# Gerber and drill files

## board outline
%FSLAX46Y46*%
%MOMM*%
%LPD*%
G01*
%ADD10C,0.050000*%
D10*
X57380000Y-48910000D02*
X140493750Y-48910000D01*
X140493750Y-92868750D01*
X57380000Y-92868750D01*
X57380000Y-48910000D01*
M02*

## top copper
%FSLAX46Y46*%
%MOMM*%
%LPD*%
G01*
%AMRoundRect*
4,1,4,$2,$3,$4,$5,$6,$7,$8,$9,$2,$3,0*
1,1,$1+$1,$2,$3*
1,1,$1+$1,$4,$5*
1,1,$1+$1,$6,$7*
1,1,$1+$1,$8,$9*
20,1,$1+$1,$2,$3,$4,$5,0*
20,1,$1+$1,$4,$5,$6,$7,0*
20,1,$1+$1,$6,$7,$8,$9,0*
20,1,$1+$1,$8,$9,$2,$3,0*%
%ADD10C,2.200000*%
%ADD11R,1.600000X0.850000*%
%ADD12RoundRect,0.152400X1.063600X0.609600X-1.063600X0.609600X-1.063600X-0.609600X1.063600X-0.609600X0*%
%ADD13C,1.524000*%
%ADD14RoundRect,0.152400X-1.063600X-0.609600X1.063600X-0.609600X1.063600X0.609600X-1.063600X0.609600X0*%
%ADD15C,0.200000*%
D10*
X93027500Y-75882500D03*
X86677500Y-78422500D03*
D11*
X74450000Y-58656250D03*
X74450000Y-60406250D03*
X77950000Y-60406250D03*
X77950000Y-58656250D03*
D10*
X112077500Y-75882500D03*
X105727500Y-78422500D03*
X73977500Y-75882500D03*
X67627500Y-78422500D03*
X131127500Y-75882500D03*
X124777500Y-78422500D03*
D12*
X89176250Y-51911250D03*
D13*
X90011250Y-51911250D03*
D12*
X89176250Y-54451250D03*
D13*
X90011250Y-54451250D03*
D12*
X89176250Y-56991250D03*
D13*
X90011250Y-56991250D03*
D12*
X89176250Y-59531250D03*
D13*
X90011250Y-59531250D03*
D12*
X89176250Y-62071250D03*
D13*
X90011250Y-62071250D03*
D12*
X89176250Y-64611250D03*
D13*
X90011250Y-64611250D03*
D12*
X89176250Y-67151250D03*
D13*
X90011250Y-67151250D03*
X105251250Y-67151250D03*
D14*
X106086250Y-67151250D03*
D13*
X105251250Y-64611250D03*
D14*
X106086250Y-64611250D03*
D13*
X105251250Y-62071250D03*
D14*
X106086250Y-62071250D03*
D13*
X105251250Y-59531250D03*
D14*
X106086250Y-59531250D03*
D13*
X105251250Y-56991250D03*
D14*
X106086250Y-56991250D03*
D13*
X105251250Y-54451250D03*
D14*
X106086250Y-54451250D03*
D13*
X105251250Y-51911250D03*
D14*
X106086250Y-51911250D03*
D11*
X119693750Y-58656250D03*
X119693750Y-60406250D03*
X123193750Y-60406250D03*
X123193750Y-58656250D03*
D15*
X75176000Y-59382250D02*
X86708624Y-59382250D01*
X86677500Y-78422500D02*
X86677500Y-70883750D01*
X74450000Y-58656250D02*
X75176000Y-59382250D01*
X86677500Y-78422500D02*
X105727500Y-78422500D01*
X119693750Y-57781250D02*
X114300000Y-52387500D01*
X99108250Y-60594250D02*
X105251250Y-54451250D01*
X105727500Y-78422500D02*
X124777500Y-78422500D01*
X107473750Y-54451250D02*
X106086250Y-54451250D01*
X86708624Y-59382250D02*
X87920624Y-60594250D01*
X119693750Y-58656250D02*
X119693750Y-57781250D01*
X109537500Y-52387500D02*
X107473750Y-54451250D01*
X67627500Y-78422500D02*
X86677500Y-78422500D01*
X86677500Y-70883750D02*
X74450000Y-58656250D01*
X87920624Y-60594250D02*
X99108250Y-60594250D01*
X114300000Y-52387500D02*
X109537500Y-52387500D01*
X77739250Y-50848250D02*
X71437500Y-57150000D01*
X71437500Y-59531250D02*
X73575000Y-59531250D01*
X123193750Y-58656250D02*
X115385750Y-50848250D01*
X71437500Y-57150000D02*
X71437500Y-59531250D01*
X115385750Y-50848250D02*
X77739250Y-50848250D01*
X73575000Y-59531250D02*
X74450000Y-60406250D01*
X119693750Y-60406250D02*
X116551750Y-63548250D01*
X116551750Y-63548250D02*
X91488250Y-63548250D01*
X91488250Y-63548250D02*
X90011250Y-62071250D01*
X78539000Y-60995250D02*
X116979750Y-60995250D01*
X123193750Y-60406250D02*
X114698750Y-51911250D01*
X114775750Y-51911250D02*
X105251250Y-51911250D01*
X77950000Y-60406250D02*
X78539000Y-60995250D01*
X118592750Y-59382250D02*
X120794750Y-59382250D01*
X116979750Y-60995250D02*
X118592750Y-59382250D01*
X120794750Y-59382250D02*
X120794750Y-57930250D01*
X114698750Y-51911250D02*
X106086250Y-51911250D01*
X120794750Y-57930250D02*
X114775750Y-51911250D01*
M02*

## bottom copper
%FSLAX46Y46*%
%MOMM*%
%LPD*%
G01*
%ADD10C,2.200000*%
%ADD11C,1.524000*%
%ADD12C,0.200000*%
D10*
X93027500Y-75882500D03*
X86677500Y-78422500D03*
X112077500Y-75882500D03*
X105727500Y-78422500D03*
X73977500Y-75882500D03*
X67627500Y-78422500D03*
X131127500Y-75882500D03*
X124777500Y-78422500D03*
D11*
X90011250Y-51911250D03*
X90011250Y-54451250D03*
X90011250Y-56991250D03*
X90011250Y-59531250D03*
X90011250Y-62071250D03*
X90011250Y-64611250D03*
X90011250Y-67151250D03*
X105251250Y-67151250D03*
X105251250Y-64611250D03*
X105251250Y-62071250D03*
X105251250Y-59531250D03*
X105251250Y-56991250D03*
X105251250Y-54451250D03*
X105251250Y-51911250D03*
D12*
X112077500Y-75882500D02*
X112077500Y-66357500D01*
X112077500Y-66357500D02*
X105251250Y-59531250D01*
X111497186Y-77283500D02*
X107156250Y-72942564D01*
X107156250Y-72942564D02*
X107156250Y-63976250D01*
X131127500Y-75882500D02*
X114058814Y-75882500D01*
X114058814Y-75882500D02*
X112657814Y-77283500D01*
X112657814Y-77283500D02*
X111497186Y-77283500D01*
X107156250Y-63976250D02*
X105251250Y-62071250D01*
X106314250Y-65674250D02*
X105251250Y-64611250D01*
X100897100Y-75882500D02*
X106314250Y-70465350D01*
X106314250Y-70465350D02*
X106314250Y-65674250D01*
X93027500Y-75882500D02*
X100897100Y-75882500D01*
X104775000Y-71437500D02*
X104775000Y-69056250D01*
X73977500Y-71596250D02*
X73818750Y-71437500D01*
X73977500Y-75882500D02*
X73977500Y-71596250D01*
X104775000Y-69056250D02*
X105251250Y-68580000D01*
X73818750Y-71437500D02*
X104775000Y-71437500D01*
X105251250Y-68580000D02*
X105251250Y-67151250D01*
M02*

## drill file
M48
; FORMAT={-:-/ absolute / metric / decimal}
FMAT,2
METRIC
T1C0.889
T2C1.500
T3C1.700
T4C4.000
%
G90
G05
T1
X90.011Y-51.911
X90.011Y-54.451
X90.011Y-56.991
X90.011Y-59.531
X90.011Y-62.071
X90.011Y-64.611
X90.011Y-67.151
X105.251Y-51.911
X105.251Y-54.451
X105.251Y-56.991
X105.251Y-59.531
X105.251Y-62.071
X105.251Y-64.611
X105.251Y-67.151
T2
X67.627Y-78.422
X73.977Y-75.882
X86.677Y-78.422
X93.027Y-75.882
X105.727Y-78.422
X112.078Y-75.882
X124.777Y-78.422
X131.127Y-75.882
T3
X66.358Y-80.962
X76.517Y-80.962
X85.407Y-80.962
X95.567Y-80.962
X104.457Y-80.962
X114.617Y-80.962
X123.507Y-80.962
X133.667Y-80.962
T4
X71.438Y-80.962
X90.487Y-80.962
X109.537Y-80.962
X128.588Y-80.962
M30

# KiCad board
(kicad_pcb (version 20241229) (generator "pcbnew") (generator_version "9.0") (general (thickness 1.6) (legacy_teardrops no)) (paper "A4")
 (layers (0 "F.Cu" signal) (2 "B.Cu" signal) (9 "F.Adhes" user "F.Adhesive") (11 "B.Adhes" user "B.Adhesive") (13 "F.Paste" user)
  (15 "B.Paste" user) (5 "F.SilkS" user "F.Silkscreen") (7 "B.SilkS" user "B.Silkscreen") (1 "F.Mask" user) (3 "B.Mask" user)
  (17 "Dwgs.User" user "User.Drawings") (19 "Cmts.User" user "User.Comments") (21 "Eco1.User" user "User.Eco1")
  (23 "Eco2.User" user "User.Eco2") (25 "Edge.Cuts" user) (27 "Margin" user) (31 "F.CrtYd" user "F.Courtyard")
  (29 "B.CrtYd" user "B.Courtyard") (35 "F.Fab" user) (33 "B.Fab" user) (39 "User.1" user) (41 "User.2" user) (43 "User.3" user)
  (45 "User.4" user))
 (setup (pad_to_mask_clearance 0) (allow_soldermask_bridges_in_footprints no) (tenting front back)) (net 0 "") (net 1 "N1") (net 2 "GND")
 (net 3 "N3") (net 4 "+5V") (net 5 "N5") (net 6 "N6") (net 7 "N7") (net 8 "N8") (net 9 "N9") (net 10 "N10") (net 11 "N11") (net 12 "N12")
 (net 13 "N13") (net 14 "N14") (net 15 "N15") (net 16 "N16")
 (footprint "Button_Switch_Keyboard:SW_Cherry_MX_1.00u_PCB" (layer "F.Cu") (at 93.0275 75.8825)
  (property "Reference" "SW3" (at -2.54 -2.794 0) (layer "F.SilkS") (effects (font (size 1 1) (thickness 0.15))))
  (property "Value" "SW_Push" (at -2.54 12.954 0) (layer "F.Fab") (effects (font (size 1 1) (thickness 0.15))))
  (pad "" np_thru_hole circle (at -7.62 5.08) (size 1.7 1.7) (drill 1.7) (layers "*.Cu" "*.Mask"))
  (pad "" np_thru_hole circle (at -2.54 5.08) (size 4 4) (drill 4) (layers "*.Cu" "*.Mask"))
  (pad "" np_thru_hole circle (at 2.54 5.08) (size 1.7 1.7) (drill 1.7) (layers "*.Cu" "*.Mask"))
  (pad "1" thru_hole circle (at 0 0) (size 2.2 2.2) (drill 1.5) (layers "*.Cu" "*.Mask") (remove_unused_layers no) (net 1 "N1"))
  (pad "2" thru_hole circle (at -6.35 2.54) (size 2.2 2.2) (drill 1.5) (layers "*.Cu" "*.Mask") (remove_unused_layers no) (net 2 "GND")))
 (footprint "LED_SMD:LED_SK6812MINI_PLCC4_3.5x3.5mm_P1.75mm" (layer "F.Cu") (at 76.2 59.53125)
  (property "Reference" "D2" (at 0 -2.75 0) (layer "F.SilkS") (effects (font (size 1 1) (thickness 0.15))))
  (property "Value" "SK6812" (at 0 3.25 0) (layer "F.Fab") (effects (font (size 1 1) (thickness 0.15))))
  (pad "1" smd rect (at -1.75 -0.875) (size 1.6 0.85) (layers "F.Cu" "F.Mask" "F.Paste") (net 2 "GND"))
  (pad "2" smd rect (at -1.75 0.875) (size 1.6 0.85) (layers "F.Cu" "F.Mask" "F.Paste") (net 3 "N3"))
  (pad "3" smd rect (at 1.75 0.875) (size 1.6 0.85) (layers "F.Cu" "F.Mask" "F.Paste") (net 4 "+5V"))
  (pad "4" smd rect (at 1.75 -0.875) (size 1.6 0.85) (layers "F.Cu" "F.Mask" "F.Paste") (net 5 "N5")))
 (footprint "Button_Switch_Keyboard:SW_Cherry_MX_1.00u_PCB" (layer "F.Cu") (at 112.0775 75.8825)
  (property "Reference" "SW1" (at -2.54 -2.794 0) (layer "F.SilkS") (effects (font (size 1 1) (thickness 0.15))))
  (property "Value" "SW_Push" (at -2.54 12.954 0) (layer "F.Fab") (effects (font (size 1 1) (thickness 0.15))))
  (pad "" np_thru_hole circle (at -7.62 5.08) (size 1.7 1.7) (drill 1.7) (layers "*.Cu" "*.Mask"))
  (pad "" np_thru_hole circle (at -2.54 5.08) (size 4 4) (drill 4) (layers "*.Cu" "*.Mask"))
  (pad "" np_thru_hole circle (at 2.54 5.08) (size 1.7 1.7) (drill 1.7) (layers "*.Cu" "*.Mask"))
  (pad "1" thru_hole circle (at 0 0) (size 2.2 2.2) (drill 1.5) (layers "*.Cu" "*.Mask") (remove_unused_layers no) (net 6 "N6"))
  (pad "2" thru_hole circle (at -6.35 2.54) (size 2.2 2.2) (drill 1.5) (layers "*.Cu" "*.Mask") (remove_unused_layers no) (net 2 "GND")))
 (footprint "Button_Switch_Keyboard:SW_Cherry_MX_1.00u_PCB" (layer "F.Cu") (at 73.9775 75.8825)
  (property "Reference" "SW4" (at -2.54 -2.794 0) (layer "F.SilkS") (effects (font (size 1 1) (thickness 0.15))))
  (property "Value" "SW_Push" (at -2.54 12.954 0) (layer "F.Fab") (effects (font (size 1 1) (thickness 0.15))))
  (pad "" np_thru_hole circle (at -7.62 5.08) (size 1.7 1.7) (drill 1.7) (layers "*.Cu" "*.Mask"))
  (pad "" np_thru_hole circle (at -2.54 5.08) (size 4 4) (drill 4) (layers "*.Cu" "*.Mask"))
  (pad "" np_thru_hole circle (at 2.54 5.08) (size 1.7 1.7) (drill 1.7) (layers "*.Cu" "*.Mask"))
  (pad "1" thru_hole circle (at 0 0) (size 2.2 2.2) (drill 1.5) (layers "*.Cu" "*.Mask") (remove_unused_layers no) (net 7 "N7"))
  (pad "2" thru_hole circle (at -6.35 2.54) (size 2.2 2.2) (drill 1.5) (layers "*.Cu" "*.Mask") (remove_unused_layers no) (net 2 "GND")))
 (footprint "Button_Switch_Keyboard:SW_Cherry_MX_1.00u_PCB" (layer "F.Cu") (at 131.1275 75.8825)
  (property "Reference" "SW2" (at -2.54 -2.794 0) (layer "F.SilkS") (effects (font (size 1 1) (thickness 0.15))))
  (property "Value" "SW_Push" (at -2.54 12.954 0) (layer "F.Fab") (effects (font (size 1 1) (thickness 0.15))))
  (pad "" np_thru_hole circle (at -7.62 5.08) (size 1.7 1.7) (drill 1.7) (layers "*.Cu" "*.Mask"))
  (pad "" np_thru_hole circle (at -2.54 5.08) (size 4 4) (drill 4) (layers "*.Cu" "*.Mask"))
  (pad "" np_thru_hole circle (at 2.54 5.08) (size 1.7 1.7) (drill 1.7) (layers "*.Cu" "*.Mask"))
  (pad "1" thru_hole circle (at 0 0) (size 2.2 2.2) (drill 1.5) (layers "*.Cu" "*.Mask") (remove_unused_layers no) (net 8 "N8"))
  (pad "2" thru_hole circle (at -6.35 2.54) (size 2.2 2.2) (drill 1.5) (layers "*.Cu" "*.Mask") (remove_unused_layers no) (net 2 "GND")))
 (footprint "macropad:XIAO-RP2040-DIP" (layer "F.Cu") (at 97.63125 59.53125)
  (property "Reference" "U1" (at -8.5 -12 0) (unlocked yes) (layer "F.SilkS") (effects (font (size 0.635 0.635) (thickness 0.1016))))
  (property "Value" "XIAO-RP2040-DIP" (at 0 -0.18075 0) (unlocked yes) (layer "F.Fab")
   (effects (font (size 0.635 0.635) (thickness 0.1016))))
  (pad "1" smd roundrect (at -8.455 -7.62 180) (size 2.432 1.524) (layers "F.Cu" "F.Mask") (roundrect_rratio 0.1) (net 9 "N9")
   (thermal_bridge_angle 45))
  (pad "1" thru_hole circle (at -7.62 -7.62 180) (size 1.524 1.524) (drill 0.889) (layers "*.Cu" "*.Mask") (remove_unused_layers no)
   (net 9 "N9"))
  (pad "2" smd roundrect (at -8.455 -5.08 180) (size 2.432 1.524) (layers "F.Cu" "F.Mask") (roundrect_rratio 0.1) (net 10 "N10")
   (thermal_bridge_angle 45))
  (pad "2" thru_hole circle (at -7.62 -5.08 180) (size 1.524 1.524) (drill 0.889) (layers "*.Cu" "*.Mask") (remove_unused_layers no)
   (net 10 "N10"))
  (pad "3" smd roundrect (at -8.455 -2.54 180) (size 2.432 1.524) (layers "F.Cu" "F.Mask") (roundrect_rratio 0.1) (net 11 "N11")
   (thermal_bridge_angle 45))
  (pad "3" thru_hole circle (at -7.62 -2.54 180) (size 1.524 1.524) (drill 0.889) (layers "*.Cu" "*.Mask") (remove_unused_layers no)
   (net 11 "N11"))
  (pad "4" smd roundrect (at -8.455 0 180) (size 2.432 1.524) (layers "F.Cu" "F.Mask") (roundrect_rratio 0.1) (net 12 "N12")
   (thermal_bridge_angle 45))
  (pad "4" thru_hole circle (at -7.62 0 180) (size 1.524 1.524) (drill 0.889) (layers "*.Cu" "*.Mask") (remove_unused_layers no)
   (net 12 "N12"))
  (pad "5" smd roundrect (at -8.455 2.54 180) (size 2.432 1.524) (layers "F.Cu" "F.Mask") (roundrect_rratio 0.1) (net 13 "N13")
   (thermal_bridge_angle 45))
  (pad "5" thru_hole circle (at -7.62 2.54 180) (size 1.524 1.524) (drill 0.889) (layers "*.Cu" "*.Mask") (remove_unused_layers no)
   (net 13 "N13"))
  (pad "6" smd roundrect (at -8.455 5.08 180) (size 2.432 1.524) (layers "F.Cu" "F.Mask") (roundrect_rratio 0.1) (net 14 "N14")
   (thermal_bridge_angle 45))
  (pad "6" thru_hole circle (at -7.62 5.08 180) (size 1.524 1.524) (drill 0.889) (layers "*.Cu" "*.Mask") (remove_unused_layers no)
   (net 14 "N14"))
  (pad "7" smd roundrect (at -8.455 7.62 180) (size 2.432 1.524) (layers "F.Cu" "F.Mask") (roundrect_rratio 0.1) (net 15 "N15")
   (thermal_bridge_angle 45))
  (pad "7" thru_hole circle (at -7.62 7.62 180) (size 1.524 1.524) (drill 0.889) (layers "*.Cu" "*.Mask") (remove_unused_layers no)
   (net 15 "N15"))
  (pad "8" thru_hole circle (at 7.62 7.62) (size 1.524 1.524) (drill 0.889) (layers "*.Cu" "*.Mask") (remove_unused_layers no) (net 7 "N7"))
  (pad "8" smd roundrect (at 8.455 7.62) (size 2.432 1.524) (layers "F.Cu" "F.Mask") (roundrect_rratio 0.1) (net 7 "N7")
   (thermal_bridge_angle 45))
  (pad "9" thru_hole circle (at 7.62 5.08) (size 1.524 1.524) (drill 0.889) (layers "*.Cu" "*.Mask") (remove_unused_layers no) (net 1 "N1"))
  (pad "9" smd roundrect (at 8.455 5.08) (size 2.432 1.524) (layers "F.Cu" "F.Mask") (roundrect_rratio 0.1) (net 1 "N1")
   (thermal_bridge_angle 45))
  (pad "10" thru_hole circle (at 7.62 2.54) (size 1.524 1.524) (drill 0.889) (layers "*.Cu" "*.Mask") (remove_unused_layers no) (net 8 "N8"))
  (pad "10" smd roundrect (at 8.455 2.54) (size 2.432 1.524) (layers "F.Cu" "F.Mask") (roundrect_rratio 0.1) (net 8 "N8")
   (thermal_bridge_angle 45))
  (pad "11" thru_hole circle (at 7.62 0) (size 1.524 1.524) (drill 0.889) (layers "*.Cu" "*.Mask") (remove_unused_layers no) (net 6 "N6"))
  (pad "11" smd roundrect (at 8.455 0) (size 2.432 1.524) (layers "F.Cu" "F.Mask") (roundrect_rratio 0.1) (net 6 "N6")
   (thermal_bridge_angle 45))
  (pad "12" thru_hole circle (at 7.62 -2.54) (size 1.524 1.524) (drill 0.889) (layers "*.Cu" "*.Mask") (remove_unused_layers no)
   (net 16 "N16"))
  (pad "12" smd roundrect (at 8.455 -2.54) (size 2.432 1.524) (layers "F.Cu" "F.Mask") (roundrect_rratio 0.1) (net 16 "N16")
   (thermal_bridge_angle 45))
  (pad "13" thru_hole circle (at 7.62 -5.08) (size 1.524 1.524) (drill 0.889) (layers "*.Cu" "*.Mask") (remove_unused_layers no)
   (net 2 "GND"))
  (pad "13" smd roundrect (at 8.455 -5.08) (size 2.432 1.524) (layers "F.Cu" "F.Mask") (roundrect_rratio 0.1) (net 2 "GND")
   (thermal_bridge_angle 45))
  (pad "14" thru_hole circle (at 7.62 -7.62) (size 1.524 1.524) (drill 0.889) (layers "*.Cu" "*.Mask") (remove_unused_layers no)
   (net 4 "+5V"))
  (pad "14" smd roundrect (at 8.455 -7.62) (size 2.432 1.524) (layers "F.Cu" "F.Mask") (roundrect_rratio 0.1) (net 4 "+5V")
   (thermal_bridge_angle 45)))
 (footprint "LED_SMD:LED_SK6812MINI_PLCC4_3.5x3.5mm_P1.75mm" (layer "F.Cu") (at 121.44375 59.53125)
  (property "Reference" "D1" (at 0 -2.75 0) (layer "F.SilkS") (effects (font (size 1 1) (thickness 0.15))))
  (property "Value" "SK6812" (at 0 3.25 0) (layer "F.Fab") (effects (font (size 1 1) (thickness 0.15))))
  (pad "1" smd rect (at -1.75 -0.875) (size 1.6 0.85) (layers "F.Cu" "F.Mask" "F.Paste") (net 2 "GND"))
  (pad "2" smd rect (at -1.75 0.875) (size 1.6 0.85) (layers "F.Cu" "F.Mask" "F.Paste") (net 13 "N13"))
  (pad "3" smd rect (at 1.75 0.875) (size 1.6 0.85) (layers "F.Cu" "F.Mask" "F.Paste") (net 4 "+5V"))
  (pad "4" smd rect (at 1.75 -0.875) (size 1.6 0.85) (layers "F.Cu" "F.Mask" "F.Paste") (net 3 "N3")))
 (gr_rect (start 57.38 48.91) (end 140.49375 92.86875) (stroke (width 0.05) (type default)) (fill no) (layer "Edge.Cuts"))
 (segment (start 75.176 59.38225) (end 86.708624 59.38225) (width 0.2) (layer "F.Cu") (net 2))
 (segment (start 86.6775 78.4225) (end 86.6775 70.88375) (width 0.2) (layer "F.Cu") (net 2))
 (segment (start 74.45 58.65625) (end 75.176 59.38225) (width 0.2) (layer "F.Cu") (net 2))
 (segment (start 86.6775 78.4225) (end 105.7275 78.4225) (width 0.2) (layer "F.Cu") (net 2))
 (segment (start 119.69375 57.78125) (end 114.3 52.3875) (width 0.2) (layer "F.Cu") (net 2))
 (segment (start 99.10825 60.59425) (end 105.25125 54.45125) (width 0.2) (layer "F.Cu") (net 2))
 (segment (start 105.7275 78.4225) (end 124.7775 78.4225) (width 0.2) (layer "F.Cu") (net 2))
 (segment (start 107.47375 54.45125) (end 106.08625 54.45125) (width 0.2) (layer "F.Cu") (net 2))
 (segment (start 86.708624 59.38225) (end 87.920624 60.59425) (width 0.2) (layer "F.Cu") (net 2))
 (segment (start 119.69375 58.65625) (end 119.69375 57.78125) (width 0.2) (layer "F.Cu") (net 2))
 (segment (start 109.5375 52.3875) (end 107.47375 54.45125) (width 0.2) (layer "F.Cu") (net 2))
 (segment (start 67.6275 78.4225) (end 86.6775 78.4225) (width 0.2) (layer "F.Cu") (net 2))
 (segment (start 86.6775 70.88375) (end 74.45 58.65625) (width 0.2) (layer "F.Cu") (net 2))
 (segment (start 87.920624 60.59425) (end 99.10825 60.59425) (width 0.2) (layer "F.Cu") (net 2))
 (segment (start 114.3 52.3875) (end 109.5375 52.3875) (width 0.2) (layer "F.Cu") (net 2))
 (segment (start 77.73925 50.84825) (end 71.4375 57.15) (width 0.2) (layer "F.Cu") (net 3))
 (segment (start 71.4375 59.53125) (end 73.575 59.53125) (width 0.2) (layer "F.Cu") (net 3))
 (segment (start 123.19375 58.65625) (end 115.38575 50.84825) (width 0.2) (layer "F.Cu") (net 3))
 (segment (start 71.4375 57.15) (end 71.4375 59.53125) (width 0.2) (layer "F.Cu") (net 3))
 (segment (start 115.38575 50.84825) (end 77.73925 50.84825) (width 0.2) (layer "F.Cu") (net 3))
 (segment (start 73.575 59.53125) (end 74.45 60.40625) (width 0.2) (layer "F.Cu") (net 3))
 (segment (start 119.69375 60.40625) (end 116.55175 63.54825) (width 0.2) (layer "F.Cu") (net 13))
 (segment (start 116.55175 63.54825) (end 91.48825 63.54825) (width 0.2) (layer "F.Cu") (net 13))
 (segment (start 91.48825 63.54825) (end 90.01125 62.07125) (width 0.2) (layer "F.Cu") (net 13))
 (segment (start 78.539 60.99525) (end 116.97975 60.99525) (width 0.2) (layer "F.Cu") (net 4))
 (segment (start 123.19375 60.40625) (end 114.69875 51.91125) (width 0.2) (layer "F.Cu") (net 4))
 (segment (start 114.77575 51.91125) (end 105.25125 51.91125) (width 0.2) (layer "F.Cu") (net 4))
 (segment (start 77.95 60.40625) (end 78.539 60.99525) (width 0.2) (layer "F.Cu") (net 4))
 (segment (start 118.59275 59.38225) (end 120.79475 59.38225) (width 0.2) (layer "F.Cu") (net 4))
 (segment (start 116.97975 60.99525) (end 118.59275 59.38225) (width 0.2) (layer "F.Cu") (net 4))
 (segment (start 120.79475 59.38225) (end 120.79475 57.93025) (width 0.2) (layer "F.Cu") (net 4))
 (segment (start 114.69875 51.91125) (end 106.08625 51.91125) (width 0.2) (layer "F.Cu") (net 4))
 (segment (start 120.79475 57.93025) (end 114.77575 51.91125) (width 0.2) (layer "F.Cu") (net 4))
 (segment (start 112.0775 75.8825) (end 112.0775 66.3575) (width 0.2) (layer "B.Cu") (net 6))
 (segment (start 112.0775 66.3575) (end 105.25125 59.53125) (width 0.2) (layer "B.Cu") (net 6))
 (segment (start 111.497186 77.2835) (end 107.15625 72.942564) (width 0.2) (layer "B.Cu") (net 8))
 (segment (start 107.15625 72.942564) (end 107.15625 63.97625) (width 0.2) (layer "B.Cu") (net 8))
 (segment (start 131.1275 75.8825) (end 114.058814 75.8825) (width 0.2) (layer "B.Cu") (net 8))
 (segment (start 114.058814 75.8825) (end 112.657814 77.2835) (width 0.2) (layer "B.Cu") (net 8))
 (segment (start 112.657814 77.2835) (end 111.497186 77.2835) (width 0.2) (layer "B.Cu") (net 8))
 (segment (start 107.15625 63.97625) (end 105.25125 62.07125) (width 0.2) (layer "B.Cu") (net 8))
 (segment (start 106.31425 65.67425) (end 105.25125 64.61125) (width 0.2) (layer "B.Cu") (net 1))
 (segment (start 100.8971 75.8825) (end 106.31425 70.46535) (width 0.2) (layer "B.Cu") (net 1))
 (segment (start 106.31425 70.46535) (end 106.31425 65.67425) (width 0.2) (layer "B.Cu") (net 1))
 (segment (start 93.0275 75.8825) (end 100.8971 75.8825) (width 0.2) (layer "B.Cu") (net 1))
 (segment (start 104.775 71.4375) (end 104.775 69.05625) (width 0.2) (layer "B.Cu") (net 7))
 (segment (start 73.9775 71.59625) (end 73.81875 71.4375) (width 0.2) (layer "B.Cu") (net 7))
 (segment (start 73.9775 75.8825) (end 73.9775 71.59625) (width 0.2) (layer "B.Cu") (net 7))
 (segment (start 104.775 69.05625) (end 105.25125 68.58) (width 0.2) (layer "B.Cu") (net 7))
 (segment (start 73.81875 71.4375) (end 104.775 71.4375) (width 0.2) (layer "B.Cu") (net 7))
 (segment (start 105.25125 68.58) (end 105.25125 67.15125) (width 0.2) (layer "B.Cu") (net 7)))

